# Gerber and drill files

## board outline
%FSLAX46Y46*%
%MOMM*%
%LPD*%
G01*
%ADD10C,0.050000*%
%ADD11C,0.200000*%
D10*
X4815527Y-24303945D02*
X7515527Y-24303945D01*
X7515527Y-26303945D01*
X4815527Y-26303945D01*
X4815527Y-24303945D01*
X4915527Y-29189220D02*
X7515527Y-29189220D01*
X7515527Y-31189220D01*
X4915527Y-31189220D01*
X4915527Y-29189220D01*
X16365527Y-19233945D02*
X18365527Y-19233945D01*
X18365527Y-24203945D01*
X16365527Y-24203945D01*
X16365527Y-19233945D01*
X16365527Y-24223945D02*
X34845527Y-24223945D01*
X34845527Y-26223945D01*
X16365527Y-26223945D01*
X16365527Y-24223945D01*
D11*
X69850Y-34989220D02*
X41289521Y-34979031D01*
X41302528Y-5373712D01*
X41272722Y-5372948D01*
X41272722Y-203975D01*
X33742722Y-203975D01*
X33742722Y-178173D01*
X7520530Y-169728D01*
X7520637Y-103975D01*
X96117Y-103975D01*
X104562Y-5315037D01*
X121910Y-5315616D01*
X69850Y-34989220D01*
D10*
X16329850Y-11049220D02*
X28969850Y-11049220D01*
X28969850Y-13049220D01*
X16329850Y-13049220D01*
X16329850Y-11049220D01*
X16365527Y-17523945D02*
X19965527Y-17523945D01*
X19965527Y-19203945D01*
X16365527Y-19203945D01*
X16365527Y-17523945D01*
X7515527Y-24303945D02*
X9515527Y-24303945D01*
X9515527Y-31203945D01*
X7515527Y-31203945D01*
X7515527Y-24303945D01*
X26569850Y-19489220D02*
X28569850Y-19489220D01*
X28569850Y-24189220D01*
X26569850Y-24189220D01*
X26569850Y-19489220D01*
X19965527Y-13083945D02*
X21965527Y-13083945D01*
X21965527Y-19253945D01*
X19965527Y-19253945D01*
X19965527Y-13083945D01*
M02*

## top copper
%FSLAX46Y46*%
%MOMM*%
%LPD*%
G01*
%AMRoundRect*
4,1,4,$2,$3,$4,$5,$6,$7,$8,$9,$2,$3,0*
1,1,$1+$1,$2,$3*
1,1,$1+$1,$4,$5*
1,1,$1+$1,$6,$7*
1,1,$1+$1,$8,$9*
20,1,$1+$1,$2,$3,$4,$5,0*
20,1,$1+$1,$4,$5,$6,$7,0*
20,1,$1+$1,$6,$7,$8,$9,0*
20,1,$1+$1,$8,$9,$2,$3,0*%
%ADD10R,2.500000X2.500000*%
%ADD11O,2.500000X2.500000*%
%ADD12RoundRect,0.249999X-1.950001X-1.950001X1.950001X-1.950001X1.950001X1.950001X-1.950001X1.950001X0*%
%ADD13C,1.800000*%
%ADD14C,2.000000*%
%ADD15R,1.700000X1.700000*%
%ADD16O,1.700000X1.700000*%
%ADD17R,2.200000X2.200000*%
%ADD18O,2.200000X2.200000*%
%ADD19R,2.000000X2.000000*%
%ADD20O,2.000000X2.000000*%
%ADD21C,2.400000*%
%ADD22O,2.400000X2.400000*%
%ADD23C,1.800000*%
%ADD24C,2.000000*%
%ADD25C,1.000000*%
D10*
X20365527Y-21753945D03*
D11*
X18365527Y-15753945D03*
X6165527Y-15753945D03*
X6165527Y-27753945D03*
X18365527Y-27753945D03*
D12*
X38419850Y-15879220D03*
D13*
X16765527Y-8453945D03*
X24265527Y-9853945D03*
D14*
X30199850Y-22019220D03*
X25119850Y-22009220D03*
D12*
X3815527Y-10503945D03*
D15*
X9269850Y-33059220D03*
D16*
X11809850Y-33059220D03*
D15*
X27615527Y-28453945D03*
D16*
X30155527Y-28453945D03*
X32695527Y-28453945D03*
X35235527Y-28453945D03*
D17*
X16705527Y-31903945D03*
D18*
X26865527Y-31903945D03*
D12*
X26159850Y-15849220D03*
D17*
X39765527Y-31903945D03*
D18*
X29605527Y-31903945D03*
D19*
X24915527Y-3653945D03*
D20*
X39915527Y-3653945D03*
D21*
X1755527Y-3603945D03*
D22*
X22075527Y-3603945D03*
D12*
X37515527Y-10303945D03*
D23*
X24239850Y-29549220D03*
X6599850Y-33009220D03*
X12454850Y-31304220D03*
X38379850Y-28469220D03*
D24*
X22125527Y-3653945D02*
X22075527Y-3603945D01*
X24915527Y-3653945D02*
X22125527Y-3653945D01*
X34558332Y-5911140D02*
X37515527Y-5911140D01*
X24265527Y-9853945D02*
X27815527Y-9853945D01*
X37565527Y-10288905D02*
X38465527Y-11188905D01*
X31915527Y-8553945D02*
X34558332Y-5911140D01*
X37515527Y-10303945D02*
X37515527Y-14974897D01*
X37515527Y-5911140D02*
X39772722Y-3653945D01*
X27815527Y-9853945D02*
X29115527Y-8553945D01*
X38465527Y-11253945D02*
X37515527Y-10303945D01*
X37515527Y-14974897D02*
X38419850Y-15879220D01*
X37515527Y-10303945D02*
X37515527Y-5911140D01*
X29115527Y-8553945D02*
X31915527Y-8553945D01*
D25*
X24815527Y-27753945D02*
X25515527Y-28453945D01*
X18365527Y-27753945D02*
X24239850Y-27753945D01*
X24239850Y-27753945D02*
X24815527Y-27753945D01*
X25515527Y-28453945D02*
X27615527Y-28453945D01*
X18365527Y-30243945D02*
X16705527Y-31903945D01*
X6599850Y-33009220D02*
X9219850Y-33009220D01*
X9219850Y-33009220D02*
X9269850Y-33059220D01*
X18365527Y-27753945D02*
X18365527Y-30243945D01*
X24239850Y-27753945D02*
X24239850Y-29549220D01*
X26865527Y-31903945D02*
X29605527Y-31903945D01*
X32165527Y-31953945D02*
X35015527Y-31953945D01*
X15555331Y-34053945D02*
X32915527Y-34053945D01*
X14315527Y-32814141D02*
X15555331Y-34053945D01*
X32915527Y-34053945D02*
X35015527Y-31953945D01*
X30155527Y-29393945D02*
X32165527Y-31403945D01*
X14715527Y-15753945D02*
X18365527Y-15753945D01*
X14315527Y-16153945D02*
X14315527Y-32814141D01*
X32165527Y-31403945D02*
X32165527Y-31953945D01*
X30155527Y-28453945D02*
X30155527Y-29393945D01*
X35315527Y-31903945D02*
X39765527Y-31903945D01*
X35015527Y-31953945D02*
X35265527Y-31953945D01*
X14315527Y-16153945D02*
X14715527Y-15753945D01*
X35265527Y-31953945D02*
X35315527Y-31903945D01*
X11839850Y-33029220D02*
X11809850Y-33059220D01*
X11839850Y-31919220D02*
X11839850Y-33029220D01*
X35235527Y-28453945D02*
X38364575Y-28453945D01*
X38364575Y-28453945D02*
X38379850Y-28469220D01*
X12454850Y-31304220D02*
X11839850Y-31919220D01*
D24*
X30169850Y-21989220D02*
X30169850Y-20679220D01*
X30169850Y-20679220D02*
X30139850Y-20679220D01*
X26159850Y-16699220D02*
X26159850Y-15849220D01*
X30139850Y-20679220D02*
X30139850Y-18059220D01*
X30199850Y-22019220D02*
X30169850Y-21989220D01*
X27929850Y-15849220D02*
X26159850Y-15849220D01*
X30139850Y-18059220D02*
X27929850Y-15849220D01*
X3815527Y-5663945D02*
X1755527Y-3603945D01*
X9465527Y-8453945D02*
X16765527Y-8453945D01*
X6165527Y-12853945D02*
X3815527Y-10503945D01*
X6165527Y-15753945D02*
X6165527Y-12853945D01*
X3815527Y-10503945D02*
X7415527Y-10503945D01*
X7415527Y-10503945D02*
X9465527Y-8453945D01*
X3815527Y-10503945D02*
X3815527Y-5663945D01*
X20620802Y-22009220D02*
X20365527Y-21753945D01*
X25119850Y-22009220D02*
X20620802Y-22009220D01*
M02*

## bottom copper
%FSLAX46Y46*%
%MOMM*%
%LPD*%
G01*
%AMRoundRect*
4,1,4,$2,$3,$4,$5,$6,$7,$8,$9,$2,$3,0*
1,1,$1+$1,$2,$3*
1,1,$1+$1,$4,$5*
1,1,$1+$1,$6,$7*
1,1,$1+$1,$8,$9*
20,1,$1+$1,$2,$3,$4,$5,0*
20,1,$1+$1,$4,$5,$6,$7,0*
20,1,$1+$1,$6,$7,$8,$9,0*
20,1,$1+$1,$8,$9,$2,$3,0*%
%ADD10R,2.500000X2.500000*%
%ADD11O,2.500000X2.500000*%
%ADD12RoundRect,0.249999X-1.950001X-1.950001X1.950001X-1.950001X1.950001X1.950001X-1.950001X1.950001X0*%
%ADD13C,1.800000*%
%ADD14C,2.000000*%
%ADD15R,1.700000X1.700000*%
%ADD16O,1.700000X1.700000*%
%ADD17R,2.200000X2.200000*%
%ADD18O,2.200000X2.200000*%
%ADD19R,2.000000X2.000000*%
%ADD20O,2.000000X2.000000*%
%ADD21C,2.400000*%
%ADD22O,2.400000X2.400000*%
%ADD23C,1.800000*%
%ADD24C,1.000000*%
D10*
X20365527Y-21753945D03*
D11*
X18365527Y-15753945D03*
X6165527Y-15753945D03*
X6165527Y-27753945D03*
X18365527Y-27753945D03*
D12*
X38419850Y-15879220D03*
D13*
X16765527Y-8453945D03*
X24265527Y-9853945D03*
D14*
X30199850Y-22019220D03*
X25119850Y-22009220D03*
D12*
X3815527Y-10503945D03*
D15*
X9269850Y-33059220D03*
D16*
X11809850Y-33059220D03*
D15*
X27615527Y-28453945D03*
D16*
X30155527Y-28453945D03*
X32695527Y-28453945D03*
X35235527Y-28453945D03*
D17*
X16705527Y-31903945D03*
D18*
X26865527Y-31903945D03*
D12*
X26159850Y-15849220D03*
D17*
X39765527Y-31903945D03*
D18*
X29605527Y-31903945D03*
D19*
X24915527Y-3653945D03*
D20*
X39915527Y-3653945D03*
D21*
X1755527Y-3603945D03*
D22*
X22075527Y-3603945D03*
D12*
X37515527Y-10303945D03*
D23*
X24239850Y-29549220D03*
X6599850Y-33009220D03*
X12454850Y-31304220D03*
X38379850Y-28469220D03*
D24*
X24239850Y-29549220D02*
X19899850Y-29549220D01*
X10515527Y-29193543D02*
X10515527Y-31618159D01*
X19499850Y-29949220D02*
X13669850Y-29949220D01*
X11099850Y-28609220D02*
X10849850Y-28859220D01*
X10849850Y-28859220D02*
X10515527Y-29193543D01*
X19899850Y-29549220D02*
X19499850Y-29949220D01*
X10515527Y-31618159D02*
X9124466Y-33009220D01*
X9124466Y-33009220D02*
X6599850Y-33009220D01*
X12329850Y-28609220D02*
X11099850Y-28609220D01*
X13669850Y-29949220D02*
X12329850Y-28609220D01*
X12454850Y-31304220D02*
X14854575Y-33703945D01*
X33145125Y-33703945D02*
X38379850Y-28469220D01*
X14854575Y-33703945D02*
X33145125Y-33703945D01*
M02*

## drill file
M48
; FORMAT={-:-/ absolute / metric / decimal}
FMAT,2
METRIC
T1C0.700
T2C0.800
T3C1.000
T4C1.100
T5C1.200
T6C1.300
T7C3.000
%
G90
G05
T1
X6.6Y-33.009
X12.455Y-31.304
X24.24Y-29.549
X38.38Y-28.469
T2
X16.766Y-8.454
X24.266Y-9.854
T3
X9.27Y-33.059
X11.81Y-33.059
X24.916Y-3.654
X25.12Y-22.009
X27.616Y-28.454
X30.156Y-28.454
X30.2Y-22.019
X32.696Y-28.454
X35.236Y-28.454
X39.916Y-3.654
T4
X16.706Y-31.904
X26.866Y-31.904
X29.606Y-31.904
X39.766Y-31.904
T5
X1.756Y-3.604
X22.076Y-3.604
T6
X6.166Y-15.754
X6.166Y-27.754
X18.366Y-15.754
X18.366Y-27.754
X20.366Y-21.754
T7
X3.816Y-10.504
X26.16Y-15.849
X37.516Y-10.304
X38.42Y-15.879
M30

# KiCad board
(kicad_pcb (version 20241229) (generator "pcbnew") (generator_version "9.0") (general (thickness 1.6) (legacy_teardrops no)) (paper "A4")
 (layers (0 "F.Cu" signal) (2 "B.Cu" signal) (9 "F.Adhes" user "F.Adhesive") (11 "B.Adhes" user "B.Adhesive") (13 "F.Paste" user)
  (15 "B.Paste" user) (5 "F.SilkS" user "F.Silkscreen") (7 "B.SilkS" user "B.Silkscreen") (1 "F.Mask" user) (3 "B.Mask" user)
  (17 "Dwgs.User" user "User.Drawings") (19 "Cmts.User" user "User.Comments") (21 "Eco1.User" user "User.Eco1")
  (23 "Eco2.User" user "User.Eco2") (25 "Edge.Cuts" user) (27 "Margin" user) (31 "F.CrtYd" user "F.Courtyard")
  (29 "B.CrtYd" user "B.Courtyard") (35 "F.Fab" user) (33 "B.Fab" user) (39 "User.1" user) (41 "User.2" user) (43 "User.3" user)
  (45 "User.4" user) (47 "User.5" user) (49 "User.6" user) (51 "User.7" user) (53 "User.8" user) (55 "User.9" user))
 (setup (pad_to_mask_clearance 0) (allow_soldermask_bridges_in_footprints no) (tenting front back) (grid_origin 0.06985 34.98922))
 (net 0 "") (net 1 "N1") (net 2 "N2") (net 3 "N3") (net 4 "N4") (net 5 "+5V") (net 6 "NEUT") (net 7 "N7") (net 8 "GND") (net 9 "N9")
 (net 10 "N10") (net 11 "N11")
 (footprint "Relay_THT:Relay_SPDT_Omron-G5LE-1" (layer "F.Cu") (at 20.365527 21.753945 -90)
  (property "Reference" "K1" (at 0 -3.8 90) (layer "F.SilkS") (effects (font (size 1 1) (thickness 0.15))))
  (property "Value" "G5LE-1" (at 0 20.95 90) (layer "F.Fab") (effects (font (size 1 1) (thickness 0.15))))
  (pad "1" thru_hole rect (at 0 0 270) (size 2.5 2.5) (drill 1.3) (layers "*.Cu" "*.Mask") (remove_unused_layers no) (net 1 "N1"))
  (pad "2" thru_hole oval (at -6 2 270) (size 2.5 2.5) (drill 1.3) (layers "*.Cu" "*.Mask") (remove_unused_layers no) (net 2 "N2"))
  (pad "3" thru_hole oval (at -6 14.2 270) (size 2.5 2.5) (drill 1.3) (layers "*.Cu" "*.Mask") (remove_unused_layers no) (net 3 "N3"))
  (pad "4" thru_hole oval (at 6 14.2 270) (size 2.5 2.5) (drill 1.3) (layers "*.Cu" "*.Mask") (remove_unused_layers no) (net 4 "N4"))
  (pad "5" thru_hole oval (at 6 2 270) (size 2.5 2.5) (drill 1.3) (layers "*.Cu" "*.Mask") (remove_unused_layers no) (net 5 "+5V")))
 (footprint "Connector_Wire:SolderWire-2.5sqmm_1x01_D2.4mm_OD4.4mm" (layer "F.Cu") (at 38.41985 15.87922)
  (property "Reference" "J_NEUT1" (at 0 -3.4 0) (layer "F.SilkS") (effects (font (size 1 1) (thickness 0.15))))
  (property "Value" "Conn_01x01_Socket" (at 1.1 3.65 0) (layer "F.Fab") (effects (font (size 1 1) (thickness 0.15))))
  (pad "1" thru_hole roundrect (at 0 0) (size 4.4 4.4) (drill 3) (layers "*.Cu" "*.Mask") (remove_unused_layers no)
   (roundrect_rratio 0.056818) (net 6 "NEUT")))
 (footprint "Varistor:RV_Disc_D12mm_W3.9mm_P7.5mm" (layer "F.Cu") (at 16.765527 8.453945)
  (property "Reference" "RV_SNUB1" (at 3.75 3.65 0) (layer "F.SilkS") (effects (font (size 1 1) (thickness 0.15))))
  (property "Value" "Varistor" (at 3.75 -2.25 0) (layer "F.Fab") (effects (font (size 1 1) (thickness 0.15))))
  (pad "1" thru_hole circle (at 0 0) (size 1.8 1.8) (drill 0.8) (layers "*.Cu" "*.Mask") (remove_unused_layers no) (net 3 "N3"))
  (pad "2" thru_hole circle (at 7.5 1.4) (size 1.8 1.8) (drill 0.8) (layers "*.Cu" "*.Mask") (remove_unused_layers no) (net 6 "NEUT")))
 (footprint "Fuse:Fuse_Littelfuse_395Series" (layer "F.Cu") (at 30.19985 22.01922 180)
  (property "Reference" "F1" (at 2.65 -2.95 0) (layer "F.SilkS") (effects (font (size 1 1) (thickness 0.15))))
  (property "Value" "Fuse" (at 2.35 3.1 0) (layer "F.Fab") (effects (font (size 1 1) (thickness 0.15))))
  (pad "1" thru_hole circle (at 0 0 180) (size 2 2) (drill 1) (layers "*.Cu" "*.Mask") (remove_unused_layers no) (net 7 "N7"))
  (pad "2" thru_hole circle (at 5.08 0.01 180) (size 2 2) (drill 1) (layers "*.Cu" "*.Mask") (remove_unused_layers no) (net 1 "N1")))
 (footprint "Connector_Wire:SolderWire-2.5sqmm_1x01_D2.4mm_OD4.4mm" (layer "F.Cu") (at 3.815527 10.503945)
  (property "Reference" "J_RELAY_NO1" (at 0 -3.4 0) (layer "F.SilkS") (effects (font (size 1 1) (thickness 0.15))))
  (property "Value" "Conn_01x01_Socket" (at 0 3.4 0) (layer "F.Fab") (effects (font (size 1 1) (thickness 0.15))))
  (pad "1" thru_hole roundrect (at 0 0) (size 4.4 4.4) (drill 3) (layers "*.Cu" "*.Mask") (remove_unused_layers no)
   (roundrect_rratio 0.056818) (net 3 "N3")))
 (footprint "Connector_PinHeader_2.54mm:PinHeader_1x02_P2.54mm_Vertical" (layer "F.Cu") (at 9.26985 33.05922 90)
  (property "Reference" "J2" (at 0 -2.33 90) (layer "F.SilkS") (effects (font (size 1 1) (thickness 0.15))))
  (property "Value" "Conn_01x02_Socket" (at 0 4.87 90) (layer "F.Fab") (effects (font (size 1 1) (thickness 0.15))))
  (pad "1" thru_hole rect (at 0 0 90) (size 1.7 1.7) (drill 1) (layers "*.Cu" "*.Mask") (remove_unused_layers no) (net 5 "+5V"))
  (pad "2" thru_hole oval (at 0 2.54 90) (size 1.7 1.7) (drill 1) (layers "*.Cu" "*.Mask") (remove_unused_layers no) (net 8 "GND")))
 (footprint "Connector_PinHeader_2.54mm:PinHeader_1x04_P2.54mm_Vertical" (layer "F.Cu") (at 27.615527 28.453945 90)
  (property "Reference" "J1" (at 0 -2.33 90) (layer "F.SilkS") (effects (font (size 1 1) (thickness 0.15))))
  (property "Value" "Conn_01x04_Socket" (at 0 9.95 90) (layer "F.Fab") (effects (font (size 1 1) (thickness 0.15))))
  (pad "1" thru_hole rect (at 0 0 90) (size 1.7 1.7) (drill 1) (layers "*.Cu" "*.Mask") (remove_unused_layers no) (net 5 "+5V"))
  (pad "2" thru_hole oval (at 0 2.54 90) (size 1.7 1.7) (drill 1) (layers "*.Cu" "*.Mask") (remove_unused_layers no) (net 2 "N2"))
  (pad "3" thru_hole oval (at 0 5.08 90) (size 1.7 1.7) (drill 1) (layers "*.Cu" "*.Mask") (remove_unused_layers no) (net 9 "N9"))
  (pad "4" thru_hole oval (at 0 7.62 90) (size 1.7 1.7) (drill 1) (layers "*.Cu" "*.Mask") (remove_unused_layers no) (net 8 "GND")))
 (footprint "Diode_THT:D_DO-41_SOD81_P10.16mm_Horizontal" (layer "F.Cu") (at 16.705527 31.903945)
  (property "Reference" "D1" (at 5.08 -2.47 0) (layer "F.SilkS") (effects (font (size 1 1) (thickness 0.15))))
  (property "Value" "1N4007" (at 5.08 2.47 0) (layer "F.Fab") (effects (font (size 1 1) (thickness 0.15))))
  (pad "1" thru_hole rect (at 0 0) (size 2.2 2.2) (drill 1.1) (layers "*.Cu" "*.Mask") (remove_unused_layers no) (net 5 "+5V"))
  (pad "2" thru_hole oval (at 10.16 0) (size 2.2 2.2) (drill 1.1) (layers "*.Cu" "*.Mask") (remove_unused_layers no) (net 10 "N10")))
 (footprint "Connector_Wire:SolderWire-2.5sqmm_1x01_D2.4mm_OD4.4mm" (layer "F.Cu") (at 26.15985 15.84922)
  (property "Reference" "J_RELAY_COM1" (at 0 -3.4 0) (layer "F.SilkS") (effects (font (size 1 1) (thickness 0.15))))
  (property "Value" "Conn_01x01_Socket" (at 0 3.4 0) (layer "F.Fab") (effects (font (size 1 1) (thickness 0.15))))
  (pad "1" thru_hole roundrect (at 0 0) (size 4.4 4.4) (drill 3) (layers "*.Cu" "*.Mask") (remove_unused_layers no)
   (roundrect_rratio 0.056818) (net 7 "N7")))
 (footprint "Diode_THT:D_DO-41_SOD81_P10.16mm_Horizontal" (layer "F.Cu") (at 39.765527 31.903945 180)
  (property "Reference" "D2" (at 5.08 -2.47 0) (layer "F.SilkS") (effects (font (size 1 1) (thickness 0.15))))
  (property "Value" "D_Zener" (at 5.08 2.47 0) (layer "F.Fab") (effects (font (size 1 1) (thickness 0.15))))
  (pad "1" thru_hole rect (at 0 0 180) (size 2.2 2.2) (drill 1.1) (layers "*.Cu" "*.Mask") (remove_unused_layers no) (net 2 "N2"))
  (pad "2" thru_hole oval (at 10.16 0 180) (size 2.2 2.2) (drill 1.1) (layers "*.Cu" "*.Mask") (remove_unused_layers no) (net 10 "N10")))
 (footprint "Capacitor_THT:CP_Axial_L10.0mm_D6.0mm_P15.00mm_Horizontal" (layer "F.Cu") (at 24.915527 3.653945)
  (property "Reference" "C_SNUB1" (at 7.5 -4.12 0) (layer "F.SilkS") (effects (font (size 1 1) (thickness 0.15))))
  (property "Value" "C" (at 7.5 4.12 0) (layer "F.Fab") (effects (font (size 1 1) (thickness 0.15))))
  (pad "1" thru_hole rect (at 0 0) (size 2 2) (drill 1) (layers "*.Cu" "*.Mask") (remove_unused_layers no) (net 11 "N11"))
  (pad "2" thru_hole oval (at 15 0) (size 2 2) (drill 1) (layers "*.Cu" "*.Mask") (remove_unused_layers no) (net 6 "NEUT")))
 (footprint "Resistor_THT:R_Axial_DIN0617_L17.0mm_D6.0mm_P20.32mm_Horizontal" (layer "F.Cu") (at 1.755527 3.603945)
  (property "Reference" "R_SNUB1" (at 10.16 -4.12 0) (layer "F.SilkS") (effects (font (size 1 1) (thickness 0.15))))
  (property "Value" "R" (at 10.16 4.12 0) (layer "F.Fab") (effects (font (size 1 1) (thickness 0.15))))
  (pad "1" thru_hole circle (at 0 0) (size 2.4 2.4) (drill 1.2) (layers "*.Cu" "*.Mask") (remove_unused_layers no) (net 3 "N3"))
  (pad "2" thru_hole oval (at 20.32 0) (size 2.4 2.4) (drill 1.2) (layers "*.Cu" "*.Mask") (remove_unused_layers no) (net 11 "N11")))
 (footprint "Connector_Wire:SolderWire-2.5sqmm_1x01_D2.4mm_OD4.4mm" (layer "F.Cu") (at 37.515527 10.303945)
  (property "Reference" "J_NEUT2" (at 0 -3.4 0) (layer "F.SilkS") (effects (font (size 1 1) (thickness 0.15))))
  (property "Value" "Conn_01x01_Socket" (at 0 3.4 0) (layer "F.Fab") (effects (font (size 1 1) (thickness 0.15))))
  (pad "1" thru_hole roundrect (at 0 0) (size 4.4 4.4) (drill 3) (layers "*.Cu" "*.Mask") (remove_unused_layers no)
   (roundrect_rratio 0.056818) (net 6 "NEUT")))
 (gr_rect (start 4.815527 24.303945) (end 7.515527 26.303945) (stroke (width 0.05) (type solid)) (fill no) (layer "Edge.Cuts"))
 (gr_rect (start 4.915527 29.18922) (end 7.515527 31.18922) (stroke (width 0.05) (type solid)) (fill no) (layer "Edge.Cuts"))
 (gr_rect (start 16.365527 19.233945) (end 18.365527 24.203945) (stroke (width 0.05) (type solid)) (fill no) (layer "Edge.Cuts"))
 (gr_rect (start 16.365527 24.223945) (end 34.845527 26.223945) (stroke (width 0.05) (type solid)) (fill no) (layer "Edge.Cuts"))
 (gr_poly
  (pts (xy 0.06985 34.98922) (xy 41.289521 34.979031) (xy 41.302528 5.373712) (xy 41.272722 5.372948) (xy 41.272722 0.203975)
   (xy 33.742722 0.203975) (xy 33.742722 0.178173) (xy 7.52053 0.169728) (xy 7.520637 0.103975) (xy 0.096117 0.103975)
   (xy 0.104562 5.315037) (xy 0.12191 5.315616))
  (stroke (width 0.2) (type solid)) (fill no) (layer "Edge.Cuts"))
 (gr_rect (start 16.32985 11.04922) (end 28.96985 13.04922) (stroke (width 0.05) (type solid)) (fill no) (layer "Edge.Cuts"))
 (gr_rect (start 16.365527 17.523945) (end 19.965527 19.203945) (stroke (width 0.05) (type solid)) (fill no) (layer "Edge.Cuts"))
 (gr_rect (start 7.515527 24.303945) (end 9.515527 31.203945) (stroke (width 0.05) (type solid)) (fill no) (layer "Edge.Cuts"))
 (gr_rect (start 26.56985 19.48922) (end 28.56985 24.18922) (stroke (width 0.05) (type default)) (fill no) (layer "Edge.Cuts"))
 (gr_rect (start 19.965527 13.083945) (end 21.965527 19.253945) (stroke (width 0.05) (type solid)) (fill no) (layer "Edge.Cuts"))
 (segment (start 22.125527 3.653945) (end 22.075527 3.603945) (width 2) (layer "F.Cu") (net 11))
 (segment (start 24.915527 3.653945) (end 22.125527 3.653945) (width 2) (layer "F.Cu") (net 11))
 (segment (start 34.558332 5.91114) (end 37.515527 5.91114) (width 2) (layer "F.Cu") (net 6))
 (segment (start 24.265527 9.853945) (end 27.815527 9.853945) (width 2) (layer "F.Cu") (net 6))
 (segment (start 37.565527 10.288905) (end 38.465527 11.188905) (width 2) (layer "F.Cu") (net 6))
 (segment (start 31.915527 8.553945) (end 34.558332 5.91114) (width 2) (layer "F.Cu") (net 6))
 (segment (start 37.515527 10.303945) (end 37.515527 14.974897) (width 2) (layer "F.Cu") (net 6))
 (segment (start 37.515527 5.91114) (end 39.772722 3.653945) (width 2) (layer "F.Cu") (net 6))
 (segment (start 27.815527 9.853945) (end 29.115527 8.553945) (width 2) (layer "F.Cu") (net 6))
 (segment (start 38.465527 11.253945) (end 37.515527 10.303945) (width 2) (layer "F.Cu") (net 6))
 (segment (start 37.515527 14.974897) (end 38.41985 15.87922) (width 2) (layer "F.Cu") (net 6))
 (segment (start 37.515527 10.303945) (end 37.515527 5.91114) (width 2) (layer "F.Cu") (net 6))
 (segment (start 29.115527 8.553945) (end 31.915527 8.553945) (width 2) (layer "F.Cu") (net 6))
 (segment (start 24.815527 27.753945) (end 25.515527 28.453945) (width 1) (layer "F.Cu") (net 5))
 (segment (start 18.365527 27.753945) (end 24.23985 27.753945) (width 1) (layer "F.Cu") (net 5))
 (segment (start 24.23985 27.753945) (end 24.815527 27.753945) (width 1) (layer "F.Cu") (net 5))
 (segment (start 25.515527 28.453945) (end 27.615527 28.453945) (width 1) (layer "F.Cu") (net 5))
 (segment (start 18.365527 30.243945) (end 16.705527 31.903945) (width 1) (layer "F.Cu") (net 5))
 (segment (start 6.59985 33.00922) (end 9.21985 33.00922) (width 1) (layer "F.Cu") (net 5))
 (segment (start 9.21985 33.00922) (end 9.26985 33.05922) (width 1) (layer "F.Cu") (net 5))
 (segment (start 18.365527 27.753945) (end 18.365527 30.243945) (width 1) (layer "F.Cu") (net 5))
 (segment (start 24.23985 27.753945) (end 24.23985 29.54922) (width 1) (layer "F.Cu") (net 5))
 (via (at 24.23985 29.54922) (size 1.8) (drill 0.7) (layers "F.Cu" "B.Cu") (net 5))
 (via (at 6.59985 33.00922) (size 1.8) (drill 0.7) (layers "F.Cu" "B.Cu") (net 5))
 (segment (start 24.23985 29.54922) (end 19.89985 29.54922) (width 1) (layer "B.Cu") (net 5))
 (segment (start 10.515527 29.193543) (end 10.515527 31.618159) (width 1) (layer "B.Cu") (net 5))
 (segment (start 19.49985 29.94922) (end 13.66985 29.94922) (width 1) (layer "B.Cu") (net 5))
 (segment (start 11.09985 28.60922) (end 10.84985 28.85922) (width 1) (layer "B.Cu") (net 5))
 (segment (start 10.84985 28.85922) (end 10.515527 29.193543) (width 1) (layer "B.Cu") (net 5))
 (segment (start 19.89985 29.54922) (end 19.49985 29.94922) (width 1) (layer "B.Cu") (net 5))
 (segment (start 10.515527 31.618159) (end 9.124466 33.00922) (width 1) (layer "B.Cu") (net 5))
 (segment (start 9.124466 33.00922) (end 6.59985 33.00922) (width 1) (layer "B.Cu") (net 5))
 (segment (start 12.32985 28.60922) (end 11.09985 28.60922) (width 1) (layer "B.Cu") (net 5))
 (segment (start 13.66985 29.94922) (end 12.32985 28.60922) (width 1) (layer "B.Cu") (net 5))
 (segment (start 26.865527 31.903945) (end 29.605527 31.903945) (width 1) (layer "F.Cu") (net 10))
 (segment (start 32.165527 31.953945) (end 35.015527 31.953945) (width 1) (layer "F.Cu") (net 2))
 (segment (start 15.555331 34.053945) (end 32.915527 34.053945) (width 1) (layer "F.Cu") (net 2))
 (segment (start 14.315527 32.814141) (end 15.555331 34.053945) (width 1) (layer "F.Cu") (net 2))
 (segment (start 32.915527 34.053945) (end 35.015527 31.953945) (width 1) (layer "F.Cu") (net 2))
 (segment (start 30.155527 29.393945) (end 32.165527 31.403945) (width 1) (layer "F.Cu") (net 2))
 (segment (start 14.715527 15.753945) (end 18.365527 15.753945) (width 1) (layer "F.Cu") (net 2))
 (segment (start 14.315527 16.153945) (end 14.315527 32.814141) (width 1) (layer "F.Cu") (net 2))
 (segment (start 32.165527 31.403945) (end 32.165527 31.953945) (width 1) (layer "F.Cu") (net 2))
 (segment (start 30.155527 28.453945) (end 30.155527 29.393945) (width 1) (layer "F.Cu") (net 2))
 (segment (start 35.315527 31.903945) (end 39.765527 31.903945) (width 1) (layer "F.Cu") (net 2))
 (segment (start 35.015527 31.953945) (end 35.265527 31.953945) (width 1) (layer "F.Cu") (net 2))
 (segment (start 14.315527 16.153945) (end 14.715527 15.753945) (width 1) (layer "F.Cu") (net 2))
 (segment (start 35.265527 31.953945) (end 35.315527 31.903945) (width 1) (layer "F.Cu") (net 2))
 (segment (start 11.83985 33.02922) (end 11.80985 33.05922) (width 1) (layer "F.Cu") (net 8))
 (segment (start 11.83985 31.91922) (end 11.83985 33.02922) (width 1) (layer "F.Cu") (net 8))
 (segment (start 35.235527 28.453945) (end 38.364575 28.453945) (width 1) (layer "F.Cu") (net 8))
 (segment (start 38.364575 28.453945) (end 38.37985 28.46922) (width 1) (layer "F.Cu") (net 8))
 (segment (start 12.45485 31.30422) (end 11.83985 31.91922) (width 1) (layer "F.Cu") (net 8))
 (via (at 12.45485 31.30422) (size 1.8) (drill 0.7) (layers "F.Cu" "B.Cu") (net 8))
 (via (at 38.37985 28.46922) (size 1.8) (drill 0.7) (layers "F.Cu" "B.Cu") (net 8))
 (segment (start 12.45485 31.30422) (end 14.854575 33.703945) (width 1) (layer "B.Cu") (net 8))
 (segment (start 33.145125 33.703945) (end 38.37985 28.46922) (width 1) (layer "B.Cu") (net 8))
 (segment (start 14.854575 33.703945) (end 33.145125 33.703945) (width 1) (layer "B.Cu") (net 8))
 (segment (start 30.16985 21.98922) (end 30.16985 20.67922) (width 2) (layer "F.Cu") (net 7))
 (segment (start 30.16985 20.67922) (end 30.13985 20.67922) (width 2) (layer "F.Cu") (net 7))
 (segment (start 26.15985 16.69922) (end 26.15985 15.84922) (width 2) (layer "F.Cu") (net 7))
 (segment (start 30.13985 20.67922) (end 30.13985 18.05922) (width 2) (layer "F.Cu") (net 7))
 (segment (start 30.19985 22.01922) (end 30.16985 21.98922) (width 2) (layer "F.Cu") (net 7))
 (segment (start 27.92985 15.84922) (end 26.15985 15.84922) (width 2) (layer "F.Cu") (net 7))
 (segment (start 30.13985 18.05922) (end 27.92985 15.84922) (width 2) (layer "F.Cu") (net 7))
 (segment (start 3.815527 5.663945) (end 1.755527 3.603945) (width 2) (layer "F.Cu") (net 3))
 (segment (start 9.465527 8.453945) (end 16.765527 8.453945) (width 2) (layer "F.Cu") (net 3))
 (segment (start 6.165527 12.853945) (end 3.815527 10.503945) (width 2) (layer "F.Cu") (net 3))
 (segment (start 6.165527 15.753945) (end 6.165527 12.853945) (width 2) (layer "F.Cu") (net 3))
 (segment (start 3.815527 10.503945) (end 7.415527 10.503945) (width 2) (layer "F.Cu") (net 3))
 (segment (start 7.415527 10.503945) (end 9.465527 8.453945) (width 2) (layer "F.Cu") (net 3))
 (segment (start 3.815527 10.503945) (end 3.815527 5.663945) (width 2) (layer "F.Cu") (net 3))
 (segment (start 20.620802 22.00922) (end 20.365527 21.753945) (width 2) (layer "F.Cu") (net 1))
 (segment (start 25.11985 22.00922) (end 20.620802 22.00922) (width 2) (layer "F.Cu") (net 1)))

